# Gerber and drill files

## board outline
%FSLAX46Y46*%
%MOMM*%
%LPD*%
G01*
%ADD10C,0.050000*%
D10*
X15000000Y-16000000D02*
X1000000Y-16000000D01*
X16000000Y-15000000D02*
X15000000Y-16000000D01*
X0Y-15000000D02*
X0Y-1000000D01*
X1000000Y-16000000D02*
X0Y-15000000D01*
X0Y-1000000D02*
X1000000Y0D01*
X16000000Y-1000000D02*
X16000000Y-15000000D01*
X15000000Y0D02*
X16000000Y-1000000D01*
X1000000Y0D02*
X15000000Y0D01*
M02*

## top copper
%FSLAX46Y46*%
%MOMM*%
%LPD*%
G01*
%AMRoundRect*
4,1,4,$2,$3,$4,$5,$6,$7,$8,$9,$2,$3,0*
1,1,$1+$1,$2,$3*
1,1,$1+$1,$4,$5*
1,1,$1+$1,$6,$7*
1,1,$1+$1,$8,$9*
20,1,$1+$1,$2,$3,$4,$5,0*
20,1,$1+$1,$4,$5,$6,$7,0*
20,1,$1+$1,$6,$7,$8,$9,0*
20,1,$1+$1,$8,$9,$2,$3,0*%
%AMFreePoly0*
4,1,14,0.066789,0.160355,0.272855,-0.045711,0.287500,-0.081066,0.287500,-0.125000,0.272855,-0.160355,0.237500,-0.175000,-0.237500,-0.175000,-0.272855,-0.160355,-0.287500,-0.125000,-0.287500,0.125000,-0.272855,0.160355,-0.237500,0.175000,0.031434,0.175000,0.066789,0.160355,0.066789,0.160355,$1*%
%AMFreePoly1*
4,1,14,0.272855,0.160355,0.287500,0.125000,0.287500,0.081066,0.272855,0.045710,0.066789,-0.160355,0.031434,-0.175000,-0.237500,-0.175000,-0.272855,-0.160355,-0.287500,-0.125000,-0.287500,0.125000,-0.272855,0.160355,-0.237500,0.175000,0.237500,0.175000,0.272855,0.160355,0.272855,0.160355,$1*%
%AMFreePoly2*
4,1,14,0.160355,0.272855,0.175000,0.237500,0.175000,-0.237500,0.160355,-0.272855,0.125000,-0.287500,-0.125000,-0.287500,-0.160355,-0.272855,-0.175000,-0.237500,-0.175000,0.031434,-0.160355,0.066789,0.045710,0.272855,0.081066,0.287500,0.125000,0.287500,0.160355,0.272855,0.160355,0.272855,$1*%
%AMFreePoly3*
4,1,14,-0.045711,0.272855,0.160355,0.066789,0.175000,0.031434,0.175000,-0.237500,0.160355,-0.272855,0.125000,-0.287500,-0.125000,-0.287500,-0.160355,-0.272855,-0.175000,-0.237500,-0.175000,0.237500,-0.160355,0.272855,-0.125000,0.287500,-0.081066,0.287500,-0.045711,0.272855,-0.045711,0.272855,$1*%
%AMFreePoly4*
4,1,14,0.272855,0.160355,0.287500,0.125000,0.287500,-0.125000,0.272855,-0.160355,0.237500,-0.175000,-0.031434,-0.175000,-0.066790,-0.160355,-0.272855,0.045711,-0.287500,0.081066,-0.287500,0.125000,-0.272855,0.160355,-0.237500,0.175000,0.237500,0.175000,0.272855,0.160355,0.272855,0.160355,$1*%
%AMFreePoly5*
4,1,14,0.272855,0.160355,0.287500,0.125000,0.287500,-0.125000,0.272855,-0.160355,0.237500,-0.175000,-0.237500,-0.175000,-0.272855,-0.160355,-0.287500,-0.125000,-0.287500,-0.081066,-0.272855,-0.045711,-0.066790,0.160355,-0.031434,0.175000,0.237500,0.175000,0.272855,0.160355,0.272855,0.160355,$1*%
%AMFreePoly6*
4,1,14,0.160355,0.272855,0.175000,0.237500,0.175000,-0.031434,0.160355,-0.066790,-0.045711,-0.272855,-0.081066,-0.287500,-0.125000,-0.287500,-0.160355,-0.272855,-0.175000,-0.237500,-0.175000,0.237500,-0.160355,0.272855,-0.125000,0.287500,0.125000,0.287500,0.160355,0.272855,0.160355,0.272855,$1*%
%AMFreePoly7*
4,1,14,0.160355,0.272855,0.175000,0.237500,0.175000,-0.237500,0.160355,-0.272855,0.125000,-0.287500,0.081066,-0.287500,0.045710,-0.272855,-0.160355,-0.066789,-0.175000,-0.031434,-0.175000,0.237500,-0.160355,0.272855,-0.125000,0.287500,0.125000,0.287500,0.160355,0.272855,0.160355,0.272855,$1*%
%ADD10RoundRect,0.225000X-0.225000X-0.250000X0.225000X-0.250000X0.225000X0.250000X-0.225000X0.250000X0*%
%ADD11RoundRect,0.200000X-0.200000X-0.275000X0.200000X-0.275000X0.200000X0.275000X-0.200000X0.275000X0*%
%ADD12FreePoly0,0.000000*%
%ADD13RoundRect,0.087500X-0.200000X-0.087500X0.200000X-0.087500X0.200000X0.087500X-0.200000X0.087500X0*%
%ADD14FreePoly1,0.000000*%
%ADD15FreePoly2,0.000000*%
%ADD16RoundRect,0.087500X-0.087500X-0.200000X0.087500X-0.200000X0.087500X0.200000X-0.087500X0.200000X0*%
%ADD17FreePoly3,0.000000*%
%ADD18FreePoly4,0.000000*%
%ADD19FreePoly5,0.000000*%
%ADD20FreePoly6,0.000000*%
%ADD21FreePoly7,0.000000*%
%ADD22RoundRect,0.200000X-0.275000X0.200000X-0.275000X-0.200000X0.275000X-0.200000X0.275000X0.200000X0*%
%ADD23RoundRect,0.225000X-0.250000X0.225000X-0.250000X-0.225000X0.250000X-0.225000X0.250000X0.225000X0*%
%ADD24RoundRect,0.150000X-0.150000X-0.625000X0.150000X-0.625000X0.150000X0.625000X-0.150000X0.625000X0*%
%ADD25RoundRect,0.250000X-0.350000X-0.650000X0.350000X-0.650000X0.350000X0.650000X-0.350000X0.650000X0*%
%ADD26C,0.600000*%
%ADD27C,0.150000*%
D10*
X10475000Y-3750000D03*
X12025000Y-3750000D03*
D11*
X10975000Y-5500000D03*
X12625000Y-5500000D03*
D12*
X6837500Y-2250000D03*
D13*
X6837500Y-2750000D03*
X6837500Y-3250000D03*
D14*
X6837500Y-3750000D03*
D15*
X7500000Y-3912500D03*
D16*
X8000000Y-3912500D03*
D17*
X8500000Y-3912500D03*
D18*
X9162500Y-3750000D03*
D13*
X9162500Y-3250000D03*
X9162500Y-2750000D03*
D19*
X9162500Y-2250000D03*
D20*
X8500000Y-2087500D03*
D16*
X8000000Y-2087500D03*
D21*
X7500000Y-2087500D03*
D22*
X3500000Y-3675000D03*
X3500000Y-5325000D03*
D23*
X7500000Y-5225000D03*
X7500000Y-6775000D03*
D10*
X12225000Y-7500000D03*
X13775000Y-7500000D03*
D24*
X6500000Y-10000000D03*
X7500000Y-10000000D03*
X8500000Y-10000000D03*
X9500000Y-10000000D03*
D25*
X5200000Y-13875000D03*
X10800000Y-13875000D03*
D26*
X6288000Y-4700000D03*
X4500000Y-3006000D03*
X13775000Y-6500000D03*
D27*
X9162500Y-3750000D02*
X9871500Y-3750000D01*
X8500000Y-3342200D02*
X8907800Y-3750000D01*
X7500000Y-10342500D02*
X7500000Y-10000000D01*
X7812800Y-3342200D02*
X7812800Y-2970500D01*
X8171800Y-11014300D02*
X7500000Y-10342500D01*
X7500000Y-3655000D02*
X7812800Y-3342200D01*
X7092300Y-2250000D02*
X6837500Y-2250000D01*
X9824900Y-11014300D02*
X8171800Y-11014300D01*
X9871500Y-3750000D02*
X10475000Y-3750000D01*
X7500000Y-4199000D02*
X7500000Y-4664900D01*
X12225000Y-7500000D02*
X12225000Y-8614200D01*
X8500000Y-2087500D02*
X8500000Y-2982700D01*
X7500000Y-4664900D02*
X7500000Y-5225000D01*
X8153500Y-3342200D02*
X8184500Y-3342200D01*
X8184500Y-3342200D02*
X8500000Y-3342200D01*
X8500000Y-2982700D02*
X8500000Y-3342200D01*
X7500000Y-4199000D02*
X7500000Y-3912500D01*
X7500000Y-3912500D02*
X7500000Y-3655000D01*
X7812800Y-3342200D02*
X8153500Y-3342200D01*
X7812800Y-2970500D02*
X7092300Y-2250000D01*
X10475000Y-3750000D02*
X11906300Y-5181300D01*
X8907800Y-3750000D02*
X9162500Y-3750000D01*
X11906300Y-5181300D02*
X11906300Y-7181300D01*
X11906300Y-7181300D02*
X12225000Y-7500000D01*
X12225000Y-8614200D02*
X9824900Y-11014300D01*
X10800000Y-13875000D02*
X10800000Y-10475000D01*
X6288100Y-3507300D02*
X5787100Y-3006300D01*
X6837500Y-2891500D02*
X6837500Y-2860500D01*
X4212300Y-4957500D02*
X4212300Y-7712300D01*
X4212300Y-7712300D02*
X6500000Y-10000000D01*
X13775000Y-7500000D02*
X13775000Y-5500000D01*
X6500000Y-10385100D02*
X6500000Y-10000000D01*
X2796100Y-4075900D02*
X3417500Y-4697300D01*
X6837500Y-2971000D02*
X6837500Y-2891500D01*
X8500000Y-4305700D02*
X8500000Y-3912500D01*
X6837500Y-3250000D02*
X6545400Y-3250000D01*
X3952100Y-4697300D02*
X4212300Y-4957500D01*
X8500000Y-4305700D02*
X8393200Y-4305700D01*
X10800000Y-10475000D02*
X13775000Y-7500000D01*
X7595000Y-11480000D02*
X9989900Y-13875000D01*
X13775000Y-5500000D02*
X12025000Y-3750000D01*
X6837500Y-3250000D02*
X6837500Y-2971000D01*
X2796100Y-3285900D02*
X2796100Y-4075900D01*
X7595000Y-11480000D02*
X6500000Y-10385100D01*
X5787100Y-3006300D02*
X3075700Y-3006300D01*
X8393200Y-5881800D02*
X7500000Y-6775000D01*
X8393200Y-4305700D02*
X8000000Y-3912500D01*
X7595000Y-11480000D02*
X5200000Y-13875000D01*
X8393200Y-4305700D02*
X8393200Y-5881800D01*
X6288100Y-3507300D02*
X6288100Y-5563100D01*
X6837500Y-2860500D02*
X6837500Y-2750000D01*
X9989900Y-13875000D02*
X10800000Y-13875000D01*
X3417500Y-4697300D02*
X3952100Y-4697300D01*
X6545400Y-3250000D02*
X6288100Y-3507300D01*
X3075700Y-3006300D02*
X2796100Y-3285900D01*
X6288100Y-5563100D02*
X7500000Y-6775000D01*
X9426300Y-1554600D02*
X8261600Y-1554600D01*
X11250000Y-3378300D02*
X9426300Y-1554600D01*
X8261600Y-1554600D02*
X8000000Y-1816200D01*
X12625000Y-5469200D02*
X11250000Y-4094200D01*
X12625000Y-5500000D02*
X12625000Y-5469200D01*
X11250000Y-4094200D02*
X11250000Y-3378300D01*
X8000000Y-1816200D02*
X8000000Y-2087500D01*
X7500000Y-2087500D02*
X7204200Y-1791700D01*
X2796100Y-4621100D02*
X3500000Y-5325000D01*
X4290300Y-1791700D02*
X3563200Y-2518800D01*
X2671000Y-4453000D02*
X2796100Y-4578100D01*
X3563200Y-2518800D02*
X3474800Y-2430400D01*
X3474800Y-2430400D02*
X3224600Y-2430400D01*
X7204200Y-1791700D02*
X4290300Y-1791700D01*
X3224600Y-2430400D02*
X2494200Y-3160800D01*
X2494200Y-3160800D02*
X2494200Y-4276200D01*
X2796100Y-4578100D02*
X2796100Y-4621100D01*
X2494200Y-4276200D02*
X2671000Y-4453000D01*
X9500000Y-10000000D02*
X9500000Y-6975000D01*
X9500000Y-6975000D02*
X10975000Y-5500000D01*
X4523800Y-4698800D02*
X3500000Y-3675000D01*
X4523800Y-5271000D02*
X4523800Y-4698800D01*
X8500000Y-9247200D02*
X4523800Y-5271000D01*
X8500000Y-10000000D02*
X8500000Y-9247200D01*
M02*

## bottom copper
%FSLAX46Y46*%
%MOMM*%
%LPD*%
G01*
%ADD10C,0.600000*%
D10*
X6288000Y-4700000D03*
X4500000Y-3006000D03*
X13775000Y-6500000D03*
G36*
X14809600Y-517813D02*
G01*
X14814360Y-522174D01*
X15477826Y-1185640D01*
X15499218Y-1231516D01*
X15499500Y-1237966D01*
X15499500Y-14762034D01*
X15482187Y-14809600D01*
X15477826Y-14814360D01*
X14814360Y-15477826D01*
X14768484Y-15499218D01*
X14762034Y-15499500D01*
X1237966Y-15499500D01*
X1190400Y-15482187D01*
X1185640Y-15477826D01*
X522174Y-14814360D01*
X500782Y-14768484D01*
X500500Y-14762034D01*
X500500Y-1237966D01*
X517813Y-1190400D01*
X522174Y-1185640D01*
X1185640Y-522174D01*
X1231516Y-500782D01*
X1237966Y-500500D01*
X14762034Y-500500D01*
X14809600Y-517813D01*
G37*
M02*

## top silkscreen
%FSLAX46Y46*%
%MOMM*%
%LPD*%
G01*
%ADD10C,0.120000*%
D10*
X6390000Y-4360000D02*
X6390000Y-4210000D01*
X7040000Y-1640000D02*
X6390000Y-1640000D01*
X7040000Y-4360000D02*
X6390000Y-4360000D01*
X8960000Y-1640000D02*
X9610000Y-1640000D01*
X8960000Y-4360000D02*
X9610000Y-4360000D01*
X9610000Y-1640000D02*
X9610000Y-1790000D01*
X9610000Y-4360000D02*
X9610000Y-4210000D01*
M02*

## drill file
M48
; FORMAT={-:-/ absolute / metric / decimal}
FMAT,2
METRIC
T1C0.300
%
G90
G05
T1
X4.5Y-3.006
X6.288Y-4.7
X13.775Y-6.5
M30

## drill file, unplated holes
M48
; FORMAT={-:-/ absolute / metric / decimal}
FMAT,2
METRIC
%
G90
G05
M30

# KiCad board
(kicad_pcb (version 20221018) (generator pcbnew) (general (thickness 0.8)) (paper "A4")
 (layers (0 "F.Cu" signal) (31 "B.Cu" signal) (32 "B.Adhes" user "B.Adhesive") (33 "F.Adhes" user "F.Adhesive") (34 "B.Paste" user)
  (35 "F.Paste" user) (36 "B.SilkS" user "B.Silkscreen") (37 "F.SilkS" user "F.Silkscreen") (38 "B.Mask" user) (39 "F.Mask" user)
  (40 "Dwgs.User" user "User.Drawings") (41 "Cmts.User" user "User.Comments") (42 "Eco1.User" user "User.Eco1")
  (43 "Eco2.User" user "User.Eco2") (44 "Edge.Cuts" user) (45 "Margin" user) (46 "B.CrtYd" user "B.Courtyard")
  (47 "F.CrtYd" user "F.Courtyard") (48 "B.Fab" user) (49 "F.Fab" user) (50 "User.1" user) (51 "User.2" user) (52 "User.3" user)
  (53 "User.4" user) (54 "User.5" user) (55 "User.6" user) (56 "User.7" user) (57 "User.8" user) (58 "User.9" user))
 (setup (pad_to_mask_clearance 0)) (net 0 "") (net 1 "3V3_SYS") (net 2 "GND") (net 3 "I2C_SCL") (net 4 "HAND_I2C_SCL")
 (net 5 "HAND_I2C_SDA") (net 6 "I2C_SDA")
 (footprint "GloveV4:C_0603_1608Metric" (layer "F.Cu") (at 11.25 3.75)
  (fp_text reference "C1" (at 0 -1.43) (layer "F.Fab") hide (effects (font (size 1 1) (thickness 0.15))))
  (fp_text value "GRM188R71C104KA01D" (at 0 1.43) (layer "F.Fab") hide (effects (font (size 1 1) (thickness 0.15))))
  (pad "1" smd roundrect (at -0.775 0) (size 0.9 0.95) (layers "F.Cu" "F.Paste" "F.Mask") (roundrect_rratio 0.25) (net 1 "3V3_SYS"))
  (pad "2" smd roundrect (at 0.775 0) (size 0.9 0.95) (layers "F.Cu" "F.Paste" "F.Mask") (roundrect_rratio 0.25) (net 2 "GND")))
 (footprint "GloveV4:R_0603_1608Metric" (layer "F.Cu") (at 11.8 5.5)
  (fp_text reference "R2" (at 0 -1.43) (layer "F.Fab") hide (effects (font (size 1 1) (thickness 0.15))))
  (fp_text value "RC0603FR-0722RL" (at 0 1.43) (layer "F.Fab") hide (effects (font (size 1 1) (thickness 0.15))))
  (pad "1" smd roundrect (at -0.825 0) (size 0.8 0.95) (layers "F.Cu" "F.Paste" "F.Mask") (roundrect_rratio 0.25) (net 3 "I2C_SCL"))
  (pad "2" smd roundrect (at 0.825 0) (size 0.8 0.95) (layers "F.Cu" "F.Paste" "F.Mask") (roundrect_rratio 0.25) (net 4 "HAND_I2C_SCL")))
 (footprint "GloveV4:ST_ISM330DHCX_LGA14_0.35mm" (layer "F.Cu") (at 8 3)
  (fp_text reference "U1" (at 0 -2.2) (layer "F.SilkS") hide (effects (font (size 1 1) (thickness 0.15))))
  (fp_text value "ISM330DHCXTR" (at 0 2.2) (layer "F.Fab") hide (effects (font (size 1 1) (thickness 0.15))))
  (fp_line (start -1.61 1.36) (end -1.61 1.21) (stroke (width 0.12) (type solid)) (layer "F.SilkS"))
  (fp_line (start -0.96 -1.36) (end -1.61 -1.36) (stroke (width 0.12) (type solid)) (layer "F.SilkS"))
  (fp_line (start -0.96 1.36) (end -1.61 1.36) (stroke (width 0.12) (type solid)) (layer "F.SilkS"))
  (fp_line (start 0.96 -1.36) (end 1.61 -1.36) (stroke (width 0.12) (type solid)) (layer "F.SilkS"))
  (fp_line (start 0.96 1.36) (end 1.61 1.36) (stroke (width 0.12) (type solid)) (layer "F.SilkS"))
  (fp_line (start 1.61 -1.36) (end 1.61 -1.21) (stroke (width 0.12) (type solid)) (layer "F.SilkS"))
  (fp_line (start 1.61 1.36) (end 1.61 1.21) (stroke (width 0.12) (type solid)) (layer "F.SilkS"))
  (pad "1" smd custom (at -1.1625 -0.75) (size 0.223223 0.223223) (layers "F.Cu" "F.Paste" "F.Mask") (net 1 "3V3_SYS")
   (thermal_bridge_angle 90) (options (clearance outline) (anchor circle)) (primitives))
  (pad "2" smd roundrect (at -1.1625 -0.25) (size 0.575 0.35) (layers "F.Cu" "F.Paste" "F.Mask") (roundrect_rratio 0.25) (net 2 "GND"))
  (pad "3" smd roundrect (at -1.1625 0.25) (size 0.575 0.35) (layers "F.Cu" "F.Paste" "F.Mask") (roundrect_rratio 0.25) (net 2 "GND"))
  (pad "4" smd custom (at -1.1625 0.75) (size 0.223223 0.223223) (layers "F.Cu" "F.Paste" "F.Mask") (thermal_bridge_angle 90)
   (options (clearance outline) (anchor circle)) (primitives))
  (pad "5" smd custom (at -0.5 0.9125) (size 0.223223 0.223223) (layers "F.Cu" "F.Paste" "F.Mask") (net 1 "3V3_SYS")
   (thermal_bridge_angle 90) (options (clearance outline) (anchor circle)) (primitives))
  (pad "6" smd roundrect (at 0 0.9125) (size 0.35 0.575) (layers "F.Cu" "F.Paste" "F.Mask") (roundrect_rratio 0.25) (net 2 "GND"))
  (pad "7" smd custom (at 0.5 0.9125) (size 0.223223 0.223223) (layers "F.Cu" "F.Paste" "F.Mask") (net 2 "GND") (thermal_bridge_angle 90)
   (options (clearance outline) (anchor circle)) (primitives))
  (pad "8" smd custom (at 1.1625 0.75) (size 0.223223 0.223223) (layers "F.Cu" "F.Paste" "F.Mask") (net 1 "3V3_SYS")
   (thermal_bridge_angle 90) (options (clearance outline) (anchor circle)) (primitives))
  (pad "9" smd roundrect (at 1.1625 0.25) (size 0.575 0.35) (layers "F.Cu" "F.Paste" "F.Mask") (roundrect_rratio 0.25))
  (pad "10" smd roundrect (at 1.1625 -0.25) (size 0.575 0.35) (layers "F.Cu" "F.Paste" "F.Mask") (roundrect_rratio 0.25))
  (pad "11" smd custom (at 1.1625 -0.75) (size 0.223223 0.223223) (layers "F.Cu" "F.Paste" "F.Mask") (thermal_bridge_angle 90)
   (options (clearance outline) (anchor circle)) (primitives))
  (pad "12" smd custom (at 0.5 -0.9125) (size 0.223223 0.223223) (layers "F.Cu" "F.Paste" "F.Mask") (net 1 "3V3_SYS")
   (thermal_bridge_angle 90) (options (clearance outline) (anchor circle)) (primitives))
  (pad "13" smd roundrect (at 0 -0.9125) (size 0.35 0.575) (layers "F.Cu" "F.Paste" "F.Mask") (roundrect_rratio 0.25) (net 4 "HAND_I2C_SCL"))
  (pad "14" smd custom (at -0.5 -0.9125) (size 0.223223 0.223223) (layers "F.Cu" "F.Paste" "F.Mask") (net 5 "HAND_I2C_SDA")
   (thermal_bridge_angle 90) (options (clearance outline) (anchor circle)) (primitives)))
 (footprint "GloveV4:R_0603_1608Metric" (layer "F.Cu") (at 3.5 4.5 -90)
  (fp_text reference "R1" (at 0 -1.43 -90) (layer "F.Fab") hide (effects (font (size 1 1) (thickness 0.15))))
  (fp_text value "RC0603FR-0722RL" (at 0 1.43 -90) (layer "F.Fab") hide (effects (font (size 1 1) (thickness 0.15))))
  (pad "1" smd roundrect (at -0.825 0 270) (size 0.8 0.95) (layers "F.Cu" "F.Paste" "F.Mask") (roundrect_rratio 0.25) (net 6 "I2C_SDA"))
  (pad "2" smd roundrect (at 0.825 0 270) (size 0.8 0.95) (layers "F.Cu" "F.Paste" "F.Mask") (roundrect_rratio 0.25) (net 5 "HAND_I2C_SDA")))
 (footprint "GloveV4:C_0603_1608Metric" (layer "F.Cu") (at 7.5 6 -90)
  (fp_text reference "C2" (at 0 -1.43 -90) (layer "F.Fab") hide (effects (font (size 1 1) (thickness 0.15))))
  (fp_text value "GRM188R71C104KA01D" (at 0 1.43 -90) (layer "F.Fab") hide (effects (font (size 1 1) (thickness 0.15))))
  (pad "1" smd roundrect (at -0.775 0 270) (size 0.9 0.95) (layers "F.Cu" "F.Paste" "F.Mask") (roundrect_rratio 0.25) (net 1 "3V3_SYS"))
  (pad "2" smd roundrect (at 0.775 0 270) (size 0.9 0.95) (layers "F.Cu" "F.Paste" "F.Mask") (roundrect_rratio 0.25) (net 2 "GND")))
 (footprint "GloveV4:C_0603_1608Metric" (layer "F.Cu") (at 13 7.5)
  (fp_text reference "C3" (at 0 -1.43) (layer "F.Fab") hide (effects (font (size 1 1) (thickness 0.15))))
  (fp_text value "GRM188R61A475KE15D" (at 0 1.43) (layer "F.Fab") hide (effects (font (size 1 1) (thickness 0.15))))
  (pad "1" smd roundrect (at -0.775 0) (size 0.9 0.95) (layers "F.Cu" "F.Paste" "F.Mask") (roundrect_rratio 0.25) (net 1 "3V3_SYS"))
  (pad "2" smd roundrect (at 0.775 0) (size 0.9 0.95) (layers "F.Cu" "F.Paste" "F.Mask") (roundrect_rratio 0.25) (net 2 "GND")))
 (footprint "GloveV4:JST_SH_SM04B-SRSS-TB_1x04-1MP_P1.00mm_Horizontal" (layer "F.Cu") (at 8 12)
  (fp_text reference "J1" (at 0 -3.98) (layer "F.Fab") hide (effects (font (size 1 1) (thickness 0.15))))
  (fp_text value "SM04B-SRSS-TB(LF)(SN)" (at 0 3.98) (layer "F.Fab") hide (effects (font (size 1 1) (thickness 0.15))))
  (pad "1" smd roundrect (at -1.5 -2) (size 0.6 1.55) (layers "F.Cu" "F.Paste" "F.Mask") (roundrect_rratio 0.25) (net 2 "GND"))
  (pad "2" smd roundrect (at -0.5 -2) (size 0.6 1.55) (layers "F.Cu" "F.Paste" "F.Mask") (roundrect_rratio 0.25) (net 1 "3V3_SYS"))
  (pad "3" smd roundrect (at 0.5 -2) (size 0.6 1.55) (layers "F.Cu" "F.Paste" "F.Mask") (roundrect_rratio 0.25) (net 6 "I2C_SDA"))
  (pad "4" smd roundrect (at 1.5 -2) (size 0.6 1.55) (layers "F.Cu" "F.Paste" "F.Mask") (roundrect_rratio 0.25) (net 3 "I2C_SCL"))
  (pad "MP" smd roundrect (at -2.8 1.875) (size 1.2 1.8) (layers "F.Cu" "F.Paste" "F.Mask") (roundrect_rratio 0.208333) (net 2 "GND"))
  (pad "MP" smd roundrect (at 2.8 1.875) (size 1.2 1.8) (layers "F.Cu" "F.Paste" "F.Mask") (roundrect_rratio 0.208333) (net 2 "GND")))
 (gr_line (start 15 16) (end 1 16) (stroke (width 0.05) (type default)) (layer "Edge.Cuts"))
 (gr_line (start 16 15) (end 15 16) (stroke (width 0.05) (type default)) (layer "Edge.Cuts"))
 (gr_line (start 0 15) (end 0 1) (stroke (width 0.05) (type default)) (layer "Edge.Cuts"))
 (gr_line (start 1 16) (end 0 15) (stroke (width 0.05) (type default)) (layer "Edge.Cuts"))
 (gr_line (start 0 1) (end 1 0) (stroke (width 0.05) (type default)) (layer "Edge.Cuts"))
 (gr_line (start 16 1) (end 16 15) (stroke (width 0.05) (type default)) (layer "Edge.Cuts"))
 (gr_line (start 15 0) (end 16 1) (stroke (width 0.05) (type default)) (layer "Edge.Cuts"))
 (gr_line (start 1 0) (end 15 0) (stroke (width 0.05) (type default)) (layer "Edge.Cuts"))
 (segment (start 9.1625 3.75) (end 9.8715 3.75) (width 0.15) (layer "F.Cu") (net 1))
 (segment (start 8.5 3.3422) (end 8.9078 3.75) (width 0.15) (layer "F.Cu") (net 1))
 (segment (start 7.5 10.3425) (end 7.5 10) (width 0.15) (layer "F.Cu") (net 1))
 (segment (start 7.8128 3.3422) (end 7.8128 2.9705) (width 0.15) (layer "F.Cu") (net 1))
 (segment (start 8.1718 11.0143) (end 7.5 10.3425) (width 0.15) (layer "F.Cu") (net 1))
 (segment (start 7.5 3.655) (end 7.8128 3.3422) (width 0.15) (layer "F.Cu") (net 1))
 (segment (start 7.0923 2.25) (end 6.8375 2.25) (width 0.15) (layer "F.Cu") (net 1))
 (segment (start 9.8249 11.0143) (end 8.1718 11.0143) (width 0.15) (layer "F.Cu") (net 1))
 (segment (start 9.8715 3.75) (end 10.475 3.75) (width 0.15) (layer "F.Cu") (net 1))
 (segment (start 7.5 4.199) (end 7.5 4.6649) (width 0.15) (layer "F.Cu") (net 1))
 (segment (start 12.225 7.5) (end 12.225 8.6142) (width 0.15) (layer "F.Cu") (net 1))
 (segment (start 8.5 2.0875) (end 8.5 2.9827) (width 0.15) (layer "F.Cu") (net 1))
 (segment (start 7.5 4.6649) (end 7.5 5.225) (width 0.15) (layer "F.Cu") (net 1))
 (segment (start 8.1535 3.3422) (end 8.1845 3.3422) (width 0.15) (layer "F.Cu") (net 1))
 (segment (start 8.1845 3.3422) (end 8.5 3.3422) (width 0.15) (layer "F.Cu") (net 1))
 (segment (start 8.5 2.9827) (end 8.5 3.3422) (width 0.15) (layer "F.Cu") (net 1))
 (segment (start 7.5 4.199) (end 7.5 3.9125) (width 0.15) (layer "F.Cu") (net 1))
 (segment (start 7.5 3.9125) (end 7.5 3.655) (width 0.15) (layer "F.Cu") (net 1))
 (segment (start 7.8128 3.3422) (end 8.1535 3.3422) (width 0.15) (layer "F.Cu") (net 1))
 (segment (start 7.8128 2.9705) (end 7.0923 2.25) (width 0.15) (layer "F.Cu") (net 1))
 (segment (start 10.475 3.75) (end 11.9063 5.1813) (width 0.15) (layer "F.Cu") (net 1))
 (segment (start 8.9078 3.75) (end 9.1625 3.75) (width 0.15) (layer "F.Cu") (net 1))
 (segment (start 11.9063 5.1813) (end 11.9063 7.1813) (width 0.15) (layer "F.Cu") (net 1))
 (segment (start 11.9063 7.1813) (end 12.225 7.5) (width 0.15) (layer "F.Cu") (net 1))
 (segment (start 12.225 8.6142) (end 9.8249 11.0143) (width 0.15) (layer "F.Cu") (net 1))
 (segment (start 10.8 13.875) (end 10.8 10.475) (width 0.15) (layer "F.Cu") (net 2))
 (segment (start 6.2881 3.5073) (end 5.7871 3.0063) (width 0.15) (layer "F.Cu") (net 2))
 (segment (start 6.8375 2.8915) (end 6.8375 2.8605) (width 0.15) (layer "F.Cu") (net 2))
 (segment (start 4.2123 4.9575) (end 4.2123 7.7123) (width 0.15) (layer "F.Cu") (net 2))
 (segment (start 4.2123 7.7123) (end 6.5 10) (width 0.15) (layer "F.Cu") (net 2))
 (segment (start 13.775 7.5) (end 13.775 5.5) (width 0.15) (layer "F.Cu") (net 2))
 (segment (start 6.5 10.3851) (end 6.5 10) (width 0.15) (layer "F.Cu") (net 2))
 (segment (start 2.7961 4.0759) (end 3.4175 4.6973) (width 0.15) (layer "F.Cu") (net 2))
 (segment (start 6.8375 2.971) (end 6.8375 2.8915) (width 0.15) (layer "F.Cu") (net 2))
 (segment (start 8.5 4.3057) (end 8.5 3.9125) (width 0.15) (layer "F.Cu") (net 2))
 (segment (start 6.8375 3.25) (end 6.5454 3.25) (width 0.15) (layer "F.Cu") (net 2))
 (segment (start 3.9521 4.6973) (end 4.2123 4.9575) (width 0.15) (layer "F.Cu") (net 2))
 (segment (start 8.5 4.3057) (end 8.3932 4.3057) (width 0.15) (layer "F.Cu") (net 2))
 (segment (start 10.8 10.475) (end 13.775 7.5) (width 0.15) (layer "F.Cu") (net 2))
 (segment (start 7.595 11.48) (end 9.9899 13.875) (width 0.15) (layer "F.Cu") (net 2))
 (segment (start 13.775 5.5) (end 12.025 3.75) (width 0.15) (layer "F.Cu") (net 2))
 (segment (start 6.8375 3.25) (end 6.8375 2.971) (width 0.15) (layer "F.Cu") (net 2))
 (segment (start 2.7961 3.2859) (end 2.7961 4.0759) (width 0.15) (layer "F.Cu") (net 2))
 (segment (start 7.595 11.48) (end 6.5 10.3851) (width 0.15) (layer "F.Cu") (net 2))
 (segment (start 5.7871 3.0063) (end 3.0757 3.0063) (width 0.15) (layer "F.Cu") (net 2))
 (segment (start 8.3932 5.8818) (end 7.5 6.775) (width 0.15) (layer "F.Cu") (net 2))
 (segment (start 8.3932 4.3057) (end 8 3.9125) (width 0.15) (layer "F.Cu") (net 2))
 (segment (start 7.595 11.48) (end 5.2 13.875) (width 0.15) (layer "F.Cu") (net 2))
 (segment (start 8.3932 4.3057) (end 8.3932 5.8818) (width 0.15) (layer "F.Cu") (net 2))
 (segment (start 6.2881 3.5073) (end 6.2881 5.5631) (width 0.15) (layer "F.Cu") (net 2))
 (segment (start 6.8375 2.8605) (end 6.8375 2.75) (width 0.15) (layer "F.Cu") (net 2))
 (segment (start 9.9899 13.875) (end 10.8 13.875) (width 0.15) (layer "F.Cu") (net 2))
 (segment (start 3.4175 4.6973) (end 3.9521 4.6973) (width 0.15) (layer "F.Cu") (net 2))
 (segment (start 6.5454 3.25) (end 6.2881 3.5073) (width 0.15) (layer "F.Cu") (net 2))
 (segment (start 3.0757 3.0063) (end 2.7961 3.2859) (width 0.15) (layer "F.Cu") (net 2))
 (segment (start 6.2881 5.5631) (end 7.5 6.775) (width 0.15) (layer "F.Cu") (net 2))
 (via (at 6.288 4.7) (size 0.6) (drill 0.3) (layers "F.Cu" "B.Cu") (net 2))
 (via (at 4.5 3.006) (size 0.6) (drill 0.3) (layers "F.Cu" "B.Cu") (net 2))
 (via (at 13.775 6.5) (size 0.6) (drill 0.3) (layers "F.Cu" "B.Cu") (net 2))
 (segment (start 9.4263 1.5546) (end 8.2616 1.5546) (width 0.15) (layer "F.Cu") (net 4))
 (segment (start 11.25 3.3783) (end 9.4263 1.5546) (width 0.15) (layer "F.Cu") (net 4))
 (segment (start 8.2616 1.5546) (end 8 1.8162) (width 0.15) (layer "F.Cu") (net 4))
 (segment (start 12.625 5.4692) (end 11.25 4.0942) (width 0.15) (layer "F.Cu") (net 4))
 (segment (start 12.625 5.5) (end 12.625 5.4692) (width 0.15) (layer "F.Cu") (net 4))
 (segment (start 11.25 4.0942) (end 11.25 3.3783) (width 0.15) (layer "F.Cu") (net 4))
 (segment (start 8 1.8162) (end 8 2.0875) (width 0.15) (layer "F.Cu") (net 4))
 (segment (start 7.5 2.0875) (end 7.2042 1.7917) (width 0.15) (layer "F.Cu") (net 5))
 (segment (start 2.7961 4.6211) (end 3.5 5.325) (width 0.15) (layer "F.Cu") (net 5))
 (segment (start 4.2903 1.7917) (end 3.5632 2.5188) (width 0.15) (layer "F.Cu") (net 5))
 (segment (start 2.671 4.453) (end 2.7961 4.5781) (width 0.15) (layer "F.Cu") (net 5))
 (segment (start 3.5632 2.5188) (end 3.4748 2.4304) (width 0.15) (layer "F.Cu") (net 5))
 (segment (start 3.4748 2.4304) (end 3.2246 2.4304) (width 0.15) (layer "F.Cu") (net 5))
 (segment (start 7.2042 1.7917) (end 4.2903 1.7917) (width 0.15) (layer "F.Cu") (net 5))
 (segment (start 3.2246 2.4304) (end 2.4942 3.1608) (width 0.15) (layer "F.Cu") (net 5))
 (segment (start 2.4942 3.1608) (end 2.4942 4.2762) (width 0.15) (layer "F.Cu") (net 5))
 (segment (start 2.7961 4.5781) (end 2.7961 4.6211) (width 0.15) (layer "F.Cu") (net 5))
 (segment (start 2.4942 4.2762) (end 2.671 4.453) (width 0.15) (layer "F.Cu") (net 5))
 (segment (start 9.5 10) (end 9.5 6.975) (width 0.15) (layer "F.Cu") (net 3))
 (segment (start 9.5 6.975) (end 10.975 5.5) (width 0.15) (layer "F.Cu") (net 3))
 (segment (start 4.5238 4.6988) (end 3.5 3.675) (width 0.15) (layer "F.Cu") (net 6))
 (segment (start 4.5238 5.271) (end 4.5238 4.6988) (width 0.15) (layer "F.Cu") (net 6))
 (segment (start 8.5 9.2472) (end 4.5238 5.271) (width 0.15) (layer "F.Cu") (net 6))
 (segment (start 8.5 10) (end 8.5 9.2472) (width 0.15) (layer "F.Cu") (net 6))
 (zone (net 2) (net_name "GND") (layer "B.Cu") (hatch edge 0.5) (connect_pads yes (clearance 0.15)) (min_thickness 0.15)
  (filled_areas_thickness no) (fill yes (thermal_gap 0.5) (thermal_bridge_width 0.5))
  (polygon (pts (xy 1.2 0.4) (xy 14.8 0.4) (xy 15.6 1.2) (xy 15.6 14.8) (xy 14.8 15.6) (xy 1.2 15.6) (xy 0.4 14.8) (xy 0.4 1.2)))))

